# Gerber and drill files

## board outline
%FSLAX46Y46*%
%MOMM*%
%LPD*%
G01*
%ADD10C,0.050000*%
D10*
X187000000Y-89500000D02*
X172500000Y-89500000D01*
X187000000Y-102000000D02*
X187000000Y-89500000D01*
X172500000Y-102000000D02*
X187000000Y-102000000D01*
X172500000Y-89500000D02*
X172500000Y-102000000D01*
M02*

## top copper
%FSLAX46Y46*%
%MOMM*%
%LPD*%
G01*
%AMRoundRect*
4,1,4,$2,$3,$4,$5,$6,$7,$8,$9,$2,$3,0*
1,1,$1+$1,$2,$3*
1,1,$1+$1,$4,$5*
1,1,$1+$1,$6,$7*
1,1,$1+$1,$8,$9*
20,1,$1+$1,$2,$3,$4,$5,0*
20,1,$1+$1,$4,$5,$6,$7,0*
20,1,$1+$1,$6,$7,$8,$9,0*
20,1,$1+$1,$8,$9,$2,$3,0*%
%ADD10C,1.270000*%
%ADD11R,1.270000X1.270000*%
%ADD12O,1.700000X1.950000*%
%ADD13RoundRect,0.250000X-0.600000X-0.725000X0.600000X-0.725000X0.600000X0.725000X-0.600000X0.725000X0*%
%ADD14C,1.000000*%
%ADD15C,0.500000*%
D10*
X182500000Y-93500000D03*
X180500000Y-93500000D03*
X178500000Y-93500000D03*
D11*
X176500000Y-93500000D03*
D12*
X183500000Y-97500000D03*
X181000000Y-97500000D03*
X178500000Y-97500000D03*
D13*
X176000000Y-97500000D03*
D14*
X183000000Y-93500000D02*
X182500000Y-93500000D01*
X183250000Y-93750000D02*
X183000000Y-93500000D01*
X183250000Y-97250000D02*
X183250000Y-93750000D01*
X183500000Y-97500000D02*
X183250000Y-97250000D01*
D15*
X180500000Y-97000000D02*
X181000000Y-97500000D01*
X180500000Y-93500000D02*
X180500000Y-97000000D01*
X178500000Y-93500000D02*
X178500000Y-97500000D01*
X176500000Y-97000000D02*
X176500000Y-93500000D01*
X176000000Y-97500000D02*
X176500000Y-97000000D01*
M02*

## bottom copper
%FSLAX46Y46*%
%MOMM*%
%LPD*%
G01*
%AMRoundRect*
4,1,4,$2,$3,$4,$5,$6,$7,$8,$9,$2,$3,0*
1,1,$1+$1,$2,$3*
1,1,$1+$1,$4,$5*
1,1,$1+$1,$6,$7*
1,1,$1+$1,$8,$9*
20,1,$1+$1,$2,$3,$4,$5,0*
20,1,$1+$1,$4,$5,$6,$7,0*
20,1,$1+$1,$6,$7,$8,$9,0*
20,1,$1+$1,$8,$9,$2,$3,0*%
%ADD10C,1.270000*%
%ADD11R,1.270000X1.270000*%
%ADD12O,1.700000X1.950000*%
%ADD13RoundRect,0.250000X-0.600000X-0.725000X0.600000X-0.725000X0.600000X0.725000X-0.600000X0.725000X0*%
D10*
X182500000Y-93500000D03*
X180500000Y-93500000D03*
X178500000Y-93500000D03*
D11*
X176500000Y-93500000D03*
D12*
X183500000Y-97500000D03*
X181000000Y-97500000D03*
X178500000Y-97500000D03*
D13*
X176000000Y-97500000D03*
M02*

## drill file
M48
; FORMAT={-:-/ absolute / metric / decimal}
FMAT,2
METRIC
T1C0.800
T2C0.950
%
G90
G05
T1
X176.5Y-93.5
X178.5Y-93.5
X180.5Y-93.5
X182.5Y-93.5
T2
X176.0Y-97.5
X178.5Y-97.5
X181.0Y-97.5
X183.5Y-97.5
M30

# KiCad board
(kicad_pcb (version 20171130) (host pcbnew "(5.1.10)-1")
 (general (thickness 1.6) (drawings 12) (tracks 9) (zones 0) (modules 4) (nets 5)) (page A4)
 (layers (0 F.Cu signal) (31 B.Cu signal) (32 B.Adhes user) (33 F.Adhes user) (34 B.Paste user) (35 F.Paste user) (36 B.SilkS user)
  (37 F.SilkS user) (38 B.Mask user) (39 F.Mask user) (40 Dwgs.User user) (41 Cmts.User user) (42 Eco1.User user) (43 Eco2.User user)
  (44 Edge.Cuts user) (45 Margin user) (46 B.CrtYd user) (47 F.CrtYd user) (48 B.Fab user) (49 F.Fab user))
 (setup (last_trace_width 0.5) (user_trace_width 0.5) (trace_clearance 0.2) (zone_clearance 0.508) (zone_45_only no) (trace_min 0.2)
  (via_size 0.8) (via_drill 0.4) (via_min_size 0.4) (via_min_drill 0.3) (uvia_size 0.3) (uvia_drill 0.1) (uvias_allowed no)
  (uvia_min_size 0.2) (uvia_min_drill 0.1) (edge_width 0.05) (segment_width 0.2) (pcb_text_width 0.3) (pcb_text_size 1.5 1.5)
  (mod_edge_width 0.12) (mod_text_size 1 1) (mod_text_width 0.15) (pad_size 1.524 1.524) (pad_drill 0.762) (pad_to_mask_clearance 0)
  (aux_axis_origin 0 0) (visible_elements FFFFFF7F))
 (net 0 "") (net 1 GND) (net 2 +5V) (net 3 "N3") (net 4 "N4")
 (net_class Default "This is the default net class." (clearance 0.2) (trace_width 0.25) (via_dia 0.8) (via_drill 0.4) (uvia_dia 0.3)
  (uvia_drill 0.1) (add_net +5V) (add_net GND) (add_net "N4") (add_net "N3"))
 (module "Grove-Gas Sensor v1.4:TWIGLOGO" (layer B.Cu) (at 184.5 94)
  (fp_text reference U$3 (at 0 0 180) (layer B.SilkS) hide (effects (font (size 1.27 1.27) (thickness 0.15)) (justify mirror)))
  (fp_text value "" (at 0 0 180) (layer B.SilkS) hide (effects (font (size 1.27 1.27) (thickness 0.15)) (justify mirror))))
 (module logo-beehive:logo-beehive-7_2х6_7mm (layer F.Cu) (at 176 93.5 270)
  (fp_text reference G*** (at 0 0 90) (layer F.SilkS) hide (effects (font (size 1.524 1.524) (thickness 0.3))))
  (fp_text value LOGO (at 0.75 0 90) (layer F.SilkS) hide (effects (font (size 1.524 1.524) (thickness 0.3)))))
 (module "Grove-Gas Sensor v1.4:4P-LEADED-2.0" (layer B.Cu) (at 179.5 93.5)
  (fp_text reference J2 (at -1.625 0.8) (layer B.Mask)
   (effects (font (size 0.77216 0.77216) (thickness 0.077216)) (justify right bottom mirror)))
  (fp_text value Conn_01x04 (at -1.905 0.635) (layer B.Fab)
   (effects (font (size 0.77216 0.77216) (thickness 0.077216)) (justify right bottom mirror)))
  (pad 4 thru_hole circle (at 3 0) (size 1.27 1.27) (drill 0.8) (layers *.Cu *.Mask) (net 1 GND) (solder_mask_margin 0.0508))
  (pad 3 thru_hole circle (at 1 0) (size 1.27 1.27) (drill 0.8) (layers *.Cu *.Mask) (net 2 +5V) (solder_mask_margin 0.0508))
  (pad 2 thru_hole circle (at -1 0) (size 1.27 1.27) (drill 0.8) (layers *.Cu *.Mask) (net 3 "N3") (solder_mask_margin 0.0508))
  (pad 1 thru_hole rect (at -3 0) (size 1.27 1.27) (drill 0.8) (layers *.Cu *.Mask) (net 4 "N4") (solder_mask_margin 0.0508)))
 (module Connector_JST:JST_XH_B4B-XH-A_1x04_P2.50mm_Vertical (layer F.Cu) (at 176 97.5)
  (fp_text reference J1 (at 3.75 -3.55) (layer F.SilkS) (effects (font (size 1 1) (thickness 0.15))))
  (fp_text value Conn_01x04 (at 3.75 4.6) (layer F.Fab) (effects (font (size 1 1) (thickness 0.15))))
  (pad 4 thru_hole oval (at 7.5 0) (size 1.7 1.95) (drill 0.95) (layers *.Cu *.Mask) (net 1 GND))
  (pad 3 thru_hole oval (at 5 0) (size 1.7 1.95) (drill 0.95) (layers *.Cu *.Mask) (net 2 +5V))
  (pad 2 thru_hole oval (at 2.5 0) (size 1.7 1.95) (drill 0.95) (layers *.Cu *.Mask) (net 3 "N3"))
  (pad 1 thru_hole roundrect (at 0 0) (size 1.7 1.95) (drill 0.95) (layers *.Cu *.Mask) (roundrect_rratio 0.147059) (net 4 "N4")))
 (gr_line (start 187 89.5) (end 172.5 89.5) (layer Edge.Cuts) (width 0.05))
 (gr_line (start 187 102) (end 187 89.5) (layer Edge.Cuts) (width 0.05))
 (gr_line (start 172.5 102) (end 187 102) (layer Edge.Cuts) (width 0.05))
 (gr_line (start 172.5 89.5) (end 172.5 102) (layer Edge.Cuts) (width 0.05))
 (segment (start 183 93.5) (end 182.5 93.5) (width 1) (layer F.Cu) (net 1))
 (segment (start 183.25 93.75) (end 183 93.5) (width 1) (layer F.Cu) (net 1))
 (segment (start 183.25 97.25) (end 183.25 93.75) (width 1) (layer F.Cu) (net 1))
 (segment (start 183.5 97.5) (end 183.25 97.25) (width 1) (layer F.Cu) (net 1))
 (segment (start 180.5 97) (end 181 97.5) (width 0.5) (layer F.Cu) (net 2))
 (segment (start 180.5 93.5) (end 180.5 97) (width 0.5) (layer F.Cu) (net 2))
 (segment (start 178.5 93.5) (end 178.5 97.5) (width 0.5) (layer F.Cu) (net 3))
 (segment (start 176.5 97) (end 176.5 93.5) (width 0.5) (layer F.Cu) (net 4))
 (segment (start 176 97.5) (end 176.5 97) (width 0.5) (layer F.Cu) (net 4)))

